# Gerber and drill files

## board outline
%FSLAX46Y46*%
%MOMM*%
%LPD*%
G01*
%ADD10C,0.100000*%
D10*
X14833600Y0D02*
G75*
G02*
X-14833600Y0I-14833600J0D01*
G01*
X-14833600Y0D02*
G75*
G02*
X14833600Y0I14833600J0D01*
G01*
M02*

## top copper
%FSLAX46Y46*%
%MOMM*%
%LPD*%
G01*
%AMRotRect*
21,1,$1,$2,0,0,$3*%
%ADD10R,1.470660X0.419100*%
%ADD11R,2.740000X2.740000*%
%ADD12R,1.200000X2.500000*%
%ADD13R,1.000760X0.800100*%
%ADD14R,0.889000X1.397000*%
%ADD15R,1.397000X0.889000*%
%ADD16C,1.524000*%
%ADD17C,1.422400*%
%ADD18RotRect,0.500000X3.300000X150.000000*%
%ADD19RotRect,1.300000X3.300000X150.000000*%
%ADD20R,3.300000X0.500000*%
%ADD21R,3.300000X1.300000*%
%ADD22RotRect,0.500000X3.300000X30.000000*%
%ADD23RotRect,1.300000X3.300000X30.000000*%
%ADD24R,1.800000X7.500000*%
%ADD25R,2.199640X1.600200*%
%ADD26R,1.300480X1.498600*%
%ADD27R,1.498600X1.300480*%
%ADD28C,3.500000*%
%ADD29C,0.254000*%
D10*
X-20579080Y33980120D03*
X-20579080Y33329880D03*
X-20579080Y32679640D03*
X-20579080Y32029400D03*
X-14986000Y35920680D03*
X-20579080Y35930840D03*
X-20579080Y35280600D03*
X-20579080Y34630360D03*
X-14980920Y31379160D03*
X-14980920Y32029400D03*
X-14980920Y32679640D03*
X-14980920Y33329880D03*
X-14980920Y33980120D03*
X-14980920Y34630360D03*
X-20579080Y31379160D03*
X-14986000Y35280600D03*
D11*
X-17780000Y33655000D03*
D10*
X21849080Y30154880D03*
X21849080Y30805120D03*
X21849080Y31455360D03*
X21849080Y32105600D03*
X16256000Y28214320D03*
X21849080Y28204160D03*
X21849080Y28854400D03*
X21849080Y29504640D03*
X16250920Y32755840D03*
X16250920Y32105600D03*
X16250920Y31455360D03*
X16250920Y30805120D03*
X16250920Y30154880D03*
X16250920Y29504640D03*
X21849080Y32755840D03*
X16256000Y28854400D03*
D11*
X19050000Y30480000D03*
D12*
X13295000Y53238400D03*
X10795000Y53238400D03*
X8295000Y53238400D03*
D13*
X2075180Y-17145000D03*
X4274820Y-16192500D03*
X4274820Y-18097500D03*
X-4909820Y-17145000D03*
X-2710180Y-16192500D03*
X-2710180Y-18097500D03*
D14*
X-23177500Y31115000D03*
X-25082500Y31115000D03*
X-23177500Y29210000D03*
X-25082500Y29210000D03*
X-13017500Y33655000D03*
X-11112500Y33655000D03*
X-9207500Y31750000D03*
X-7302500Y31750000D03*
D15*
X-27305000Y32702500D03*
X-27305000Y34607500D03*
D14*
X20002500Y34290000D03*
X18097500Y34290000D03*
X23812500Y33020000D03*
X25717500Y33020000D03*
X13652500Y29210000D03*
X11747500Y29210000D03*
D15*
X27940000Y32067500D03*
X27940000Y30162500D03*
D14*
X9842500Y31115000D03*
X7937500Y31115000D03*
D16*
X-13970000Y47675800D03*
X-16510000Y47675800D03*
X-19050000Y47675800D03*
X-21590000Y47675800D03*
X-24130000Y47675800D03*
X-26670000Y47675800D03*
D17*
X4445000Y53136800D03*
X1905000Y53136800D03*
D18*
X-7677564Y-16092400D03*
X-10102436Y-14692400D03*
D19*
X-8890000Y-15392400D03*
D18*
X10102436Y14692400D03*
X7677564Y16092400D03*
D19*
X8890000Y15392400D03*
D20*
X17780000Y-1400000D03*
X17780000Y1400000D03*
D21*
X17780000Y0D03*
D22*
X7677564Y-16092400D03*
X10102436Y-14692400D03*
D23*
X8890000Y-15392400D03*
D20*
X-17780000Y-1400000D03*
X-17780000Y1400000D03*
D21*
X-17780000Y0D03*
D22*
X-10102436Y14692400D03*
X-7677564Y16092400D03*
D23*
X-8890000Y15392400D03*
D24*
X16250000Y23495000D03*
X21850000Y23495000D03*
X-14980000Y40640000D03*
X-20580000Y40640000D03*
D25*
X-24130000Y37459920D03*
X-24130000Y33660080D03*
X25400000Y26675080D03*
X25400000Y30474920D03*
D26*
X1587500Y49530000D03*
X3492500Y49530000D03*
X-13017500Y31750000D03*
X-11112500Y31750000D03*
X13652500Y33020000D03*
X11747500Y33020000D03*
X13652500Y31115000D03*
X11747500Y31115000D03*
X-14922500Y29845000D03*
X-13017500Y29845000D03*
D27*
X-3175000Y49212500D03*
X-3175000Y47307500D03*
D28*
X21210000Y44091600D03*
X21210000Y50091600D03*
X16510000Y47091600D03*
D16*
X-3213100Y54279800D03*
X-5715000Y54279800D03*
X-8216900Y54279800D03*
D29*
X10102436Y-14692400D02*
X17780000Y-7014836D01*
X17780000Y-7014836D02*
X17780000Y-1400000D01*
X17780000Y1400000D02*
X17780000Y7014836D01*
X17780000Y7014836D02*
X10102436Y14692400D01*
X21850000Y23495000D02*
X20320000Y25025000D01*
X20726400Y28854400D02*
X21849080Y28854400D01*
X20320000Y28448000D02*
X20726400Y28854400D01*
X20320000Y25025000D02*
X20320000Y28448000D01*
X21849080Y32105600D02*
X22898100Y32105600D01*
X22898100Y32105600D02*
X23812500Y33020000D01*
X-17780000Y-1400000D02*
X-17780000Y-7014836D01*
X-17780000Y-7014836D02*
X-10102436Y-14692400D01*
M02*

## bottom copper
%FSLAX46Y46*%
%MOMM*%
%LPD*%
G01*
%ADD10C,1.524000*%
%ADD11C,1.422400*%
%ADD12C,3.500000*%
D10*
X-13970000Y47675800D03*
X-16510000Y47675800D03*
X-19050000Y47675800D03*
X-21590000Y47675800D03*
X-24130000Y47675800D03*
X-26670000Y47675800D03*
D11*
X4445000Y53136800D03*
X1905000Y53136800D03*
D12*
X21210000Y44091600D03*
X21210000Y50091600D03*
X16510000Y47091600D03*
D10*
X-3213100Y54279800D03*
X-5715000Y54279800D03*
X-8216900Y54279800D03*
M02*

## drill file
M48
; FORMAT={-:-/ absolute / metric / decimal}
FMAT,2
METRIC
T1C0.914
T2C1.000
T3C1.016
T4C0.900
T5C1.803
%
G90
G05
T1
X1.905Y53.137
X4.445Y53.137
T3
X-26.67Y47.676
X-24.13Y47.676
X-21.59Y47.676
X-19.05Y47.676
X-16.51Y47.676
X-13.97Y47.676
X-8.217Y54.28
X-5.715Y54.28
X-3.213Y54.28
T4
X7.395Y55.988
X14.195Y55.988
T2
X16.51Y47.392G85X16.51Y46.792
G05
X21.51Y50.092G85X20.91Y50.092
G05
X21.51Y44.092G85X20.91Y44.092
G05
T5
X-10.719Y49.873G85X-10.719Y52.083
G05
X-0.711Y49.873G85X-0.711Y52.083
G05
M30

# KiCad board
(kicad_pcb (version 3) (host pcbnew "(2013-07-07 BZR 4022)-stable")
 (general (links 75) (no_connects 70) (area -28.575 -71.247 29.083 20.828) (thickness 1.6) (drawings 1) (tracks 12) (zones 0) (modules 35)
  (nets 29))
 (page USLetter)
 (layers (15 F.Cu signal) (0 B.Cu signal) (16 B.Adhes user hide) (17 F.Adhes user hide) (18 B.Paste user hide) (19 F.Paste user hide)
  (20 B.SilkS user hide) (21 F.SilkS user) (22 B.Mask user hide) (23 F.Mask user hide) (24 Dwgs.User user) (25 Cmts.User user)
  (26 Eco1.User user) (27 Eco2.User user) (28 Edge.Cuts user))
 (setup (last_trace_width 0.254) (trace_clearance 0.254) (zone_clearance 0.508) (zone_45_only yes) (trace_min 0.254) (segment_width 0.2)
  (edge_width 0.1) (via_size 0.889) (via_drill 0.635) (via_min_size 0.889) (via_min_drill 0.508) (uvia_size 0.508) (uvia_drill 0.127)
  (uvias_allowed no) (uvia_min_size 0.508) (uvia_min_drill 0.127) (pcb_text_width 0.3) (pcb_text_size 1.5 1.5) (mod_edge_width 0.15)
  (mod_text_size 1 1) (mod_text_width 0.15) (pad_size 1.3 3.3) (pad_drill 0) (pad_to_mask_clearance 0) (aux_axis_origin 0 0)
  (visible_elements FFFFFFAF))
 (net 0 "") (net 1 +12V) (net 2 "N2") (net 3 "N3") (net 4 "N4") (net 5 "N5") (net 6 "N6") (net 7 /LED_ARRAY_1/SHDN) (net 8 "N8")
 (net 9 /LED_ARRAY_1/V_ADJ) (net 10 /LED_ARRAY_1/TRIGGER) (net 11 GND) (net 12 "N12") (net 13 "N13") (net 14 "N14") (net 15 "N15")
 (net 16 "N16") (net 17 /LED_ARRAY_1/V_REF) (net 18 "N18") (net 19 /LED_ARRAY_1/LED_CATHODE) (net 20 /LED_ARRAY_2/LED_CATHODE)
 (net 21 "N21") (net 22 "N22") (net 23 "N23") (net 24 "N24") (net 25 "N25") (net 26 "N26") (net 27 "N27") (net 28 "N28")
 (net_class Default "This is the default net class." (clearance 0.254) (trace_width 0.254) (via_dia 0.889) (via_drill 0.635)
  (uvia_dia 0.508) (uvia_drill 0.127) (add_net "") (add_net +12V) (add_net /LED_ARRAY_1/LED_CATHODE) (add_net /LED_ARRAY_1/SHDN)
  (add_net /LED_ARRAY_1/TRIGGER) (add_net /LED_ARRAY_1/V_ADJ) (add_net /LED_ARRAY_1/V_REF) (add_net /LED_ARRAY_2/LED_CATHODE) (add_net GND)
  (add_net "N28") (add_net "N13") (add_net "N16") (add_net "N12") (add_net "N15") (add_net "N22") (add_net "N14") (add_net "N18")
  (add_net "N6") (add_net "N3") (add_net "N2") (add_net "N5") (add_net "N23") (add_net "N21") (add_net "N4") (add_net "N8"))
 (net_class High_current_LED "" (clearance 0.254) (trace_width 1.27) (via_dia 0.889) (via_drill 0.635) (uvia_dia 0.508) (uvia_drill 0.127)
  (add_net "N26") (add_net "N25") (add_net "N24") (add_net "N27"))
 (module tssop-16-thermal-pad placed (layer F.Cu) (at -17.78 -33.655 270)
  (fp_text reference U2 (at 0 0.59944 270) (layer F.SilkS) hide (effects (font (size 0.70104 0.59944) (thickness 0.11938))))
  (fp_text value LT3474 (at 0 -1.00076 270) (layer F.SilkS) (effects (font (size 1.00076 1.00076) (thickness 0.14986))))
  (pad 4 smd rect (at -0.32512 2.79908 270) (size 0.4191 1.47066) (layers F.Cu F.Paste F.Mask) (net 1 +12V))
  (pad 5 smd rect (at 0.32512 2.79908 270) (size 0.4191 1.47066) (layers F.Cu F.Paste F.Mask) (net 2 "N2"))
  (pad 6 smd rect (at 0.97536 2.79908 270) (size 0.4191 1.47066) (layers F.Cu F.Paste F.Mask) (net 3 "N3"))
  (pad 7 smd rect (at 1.6256 2.79908 270) (size 0.4191 1.47066) (layers F.Cu F.Paste F.Mask) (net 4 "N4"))
  (pad 16 smd rect (at -2.26568 -2.794 270) (size 0.4191 1.47066) (layers F.Cu F.Paste F.Mask))
  (pad 1 smd rect (at -2.27584 2.79908 270) (size 0.4191 1.47066) (layers F.Cu F.Paste F.Mask))
  (pad 2 smd rect (at -1.6256 2.79908 270) (size 0.4191 1.47066) (layers F.Cu F.Paste F.Mask) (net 4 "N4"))
  (pad 3 smd rect (at -0.97536 2.79908 270) (size 0.4191 1.47066) (layers F.Cu F.Paste F.Mask) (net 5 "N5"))
  (pad 9 smd rect (at 2.27584 -2.79908 270) (size 0.4191 1.47066) (layers F.Cu F.Paste F.Mask) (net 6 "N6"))
  (pad 10 smd rect (at 1.6256 -2.79908 270) (size 0.4191 1.47066) (layers F.Cu F.Paste F.Mask) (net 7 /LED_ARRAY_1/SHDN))
  (pad 11 smd rect (at 0.97536 -2.79908 270) (size 0.4191 1.47066) (layers F.Cu F.Paste F.Mask))
  (pad 12 smd rect (at 0.32512 -2.79908 270) (size 0.4191 1.47066) (layers F.Cu F.Paste F.Mask) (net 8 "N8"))
  (pad 13 smd rect (at -0.32512 -2.79908 270) (size 0.4191 1.47066) (layers F.Cu F.Paste F.Mask) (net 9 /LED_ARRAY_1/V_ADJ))
  (pad 14 smd rect (at -0.97536 -2.79908 270) (size 0.4191 1.47066) (layers F.Cu F.Paste F.Mask) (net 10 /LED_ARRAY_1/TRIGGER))
  (pad 8 smd rect (at 2.27584 2.79908 270) (size 0.4191 1.47066) (layers F.Cu F.Paste F.Mask) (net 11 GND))
  (pad 15 smd rect (at -1.6256 -2.794 270) (size 0.4191 1.47066) (layers F.Cu F.Paste F.Mask) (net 11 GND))
  (pad 17 smd rect (at 0 0 270) (size 2.74 2.74) (layers F.Cu F.Paste F.Mask) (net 11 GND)))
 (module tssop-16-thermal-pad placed (layer F.Cu) (at 19.05 -30.48 90)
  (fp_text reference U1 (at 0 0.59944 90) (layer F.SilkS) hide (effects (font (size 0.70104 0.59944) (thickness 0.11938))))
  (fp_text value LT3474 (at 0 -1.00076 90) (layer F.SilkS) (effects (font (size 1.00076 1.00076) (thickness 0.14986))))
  (pad 4 smd rect (at -0.32512 2.79908 90) (size 0.4191 1.47066) (layers F.Cu F.Paste F.Mask) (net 1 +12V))
  (pad 5 smd rect (at 0.32512 2.79908 90) (size 0.4191 1.47066) (layers F.Cu F.Paste F.Mask) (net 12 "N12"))
  (pad 6 smd rect (at 0.97536 2.79908 90) (size 0.4191 1.47066) (layers F.Cu F.Paste F.Mask) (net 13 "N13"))
  (pad 7 smd rect (at 1.6256 2.79908 90) (size 0.4191 1.47066) (layers F.Cu F.Paste F.Mask) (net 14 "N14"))
  (pad 16 smd rect (at -2.26568 -2.794 90) (size 0.4191 1.47066) (layers F.Cu F.Paste F.Mask))
  (pad 1 smd rect (at -2.27584 2.79908 90) (size 0.4191 1.47066) (layers F.Cu F.Paste F.Mask))
  (pad 2 smd rect (at -1.6256 2.79908 90) (size 0.4191 1.47066) (layers F.Cu F.Paste F.Mask) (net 14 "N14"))
  (pad 3 smd rect (at -0.97536 2.79908 90) (size 0.4191 1.47066) (layers F.Cu F.Paste F.Mask) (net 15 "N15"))
  (pad 9 smd rect (at 2.27584 -2.79908 90) (size 0.4191 1.47066) (layers F.Cu F.Paste F.Mask) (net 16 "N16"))
  (pad 10 smd rect (at 1.6256 -2.79908 90) (size 0.4191 1.47066) (layers F.Cu F.Paste F.Mask) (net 7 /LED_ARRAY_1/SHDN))
  (pad 11 smd rect (at 0.97536 -2.79908 90) (size 0.4191 1.47066) (layers F.Cu F.Paste F.Mask) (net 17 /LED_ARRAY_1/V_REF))
  (pad 12 smd rect (at 0.32512 -2.79908 90) (size 0.4191 1.47066) (layers F.Cu F.Paste F.Mask) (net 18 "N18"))
  (pad 13 smd rect (at -0.32512 -2.79908 90) (size 0.4191 1.47066) (layers F.Cu F.Paste F.Mask) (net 9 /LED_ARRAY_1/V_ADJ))
  (pad 14 smd rect (at -0.97536 -2.79908 90) (size 0.4191 1.47066) (layers F.Cu F.Paste F.Mask) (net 10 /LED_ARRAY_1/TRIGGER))
  (pad 8 smd rect (at 2.27584 2.79908 90) (size 0.4191 1.47066) (layers F.Cu F.Paste F.Mask) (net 11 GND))
  (pad 15 smd rect (at -1.6256 -2.794 90) (size 0.4191 1.47066) (layers F.Cu F.Paste F.Mask) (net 11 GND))
  (pad 17 smd rect (at 0 0 90) (size 2.74 2.74) (layers F.Cu F.Paste F.Mask) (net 11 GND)))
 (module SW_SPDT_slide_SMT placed (layer F.Cu) (at 10.795 -53.2384 180)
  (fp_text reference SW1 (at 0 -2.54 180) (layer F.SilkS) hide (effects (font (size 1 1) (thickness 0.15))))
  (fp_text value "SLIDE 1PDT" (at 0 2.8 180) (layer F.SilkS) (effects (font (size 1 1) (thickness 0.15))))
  (pad 1 smd rect (at -2.5 0 180) (size 1.2 2.5) (layers F.Cu F.Paste F.Mask) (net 11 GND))
  (pad 2 smd rect (at 0 0 180) (size 1.2 2.5) (layers F.Cu F.Paste F.Mask) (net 7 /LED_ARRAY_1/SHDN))
  (pad 3 smd rect (at 2.5 0 180) (size 1.2 2.5) (layers F.Cu F.Paste F.Mask) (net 1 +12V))
  (pad "" np_thru_hole circle (at 3.4 2.75 180) (size 0.9 0.9) (drill 0.9) (layers *.Cu *.Mask F.SilkS))
  (pad "" np_thru_hole circle (at -3.4 2.75 180) (size 0.9 0.9) (drill 0.9) (layers *.Cu *.Mask F.SilkS)))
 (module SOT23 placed (layer F.Cu) (at 3.175 17.145 90)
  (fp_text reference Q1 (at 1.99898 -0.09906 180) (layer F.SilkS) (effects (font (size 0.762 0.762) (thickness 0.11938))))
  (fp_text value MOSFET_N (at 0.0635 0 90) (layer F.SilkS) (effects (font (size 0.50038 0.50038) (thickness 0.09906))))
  (pad 3 smd rect (at 0 -1.09982 90) (size 0.8001 1.00076) (layers F.Cu F.Paste F.Mask) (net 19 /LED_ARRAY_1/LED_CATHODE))
  (pad 2 smd rect (at 0.9525 1.09982 90) (size 0.8001 1.00076) (layers F.Cu F.Paste F.Mask) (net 11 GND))
  (pad 1 smd rect (at -0.9525 1.09982 90) (size 0.8001 1.00076) (layers F.Cu F.Paste F.Mask) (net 10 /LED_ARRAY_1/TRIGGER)))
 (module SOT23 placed (layer F.Cu) (at -3.81 17.145 90)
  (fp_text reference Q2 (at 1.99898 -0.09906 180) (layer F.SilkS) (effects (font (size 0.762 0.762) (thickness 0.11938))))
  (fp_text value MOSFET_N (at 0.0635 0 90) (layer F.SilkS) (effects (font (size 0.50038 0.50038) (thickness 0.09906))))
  (pad 3 smd rect (at 0 -1.09982 90) (size 0.8001 1.00076) (layers F.Cu F.Paste F.Mask) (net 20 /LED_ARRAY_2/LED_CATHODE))
  (pad 2 smd rect (at 0.9525 1.09982 90) (size 0.8001 1.00076) (layers F.Cu F.Paste F.Mask) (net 11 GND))
  (pad 1 smd rect (at -0.9525 1.09982 90) (size 0.8001 1.00076) (layers F.Cu F.Paste F.Mask) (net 10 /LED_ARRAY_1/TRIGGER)))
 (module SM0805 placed (layer F.Cu) (at -24.13 -31.115 180)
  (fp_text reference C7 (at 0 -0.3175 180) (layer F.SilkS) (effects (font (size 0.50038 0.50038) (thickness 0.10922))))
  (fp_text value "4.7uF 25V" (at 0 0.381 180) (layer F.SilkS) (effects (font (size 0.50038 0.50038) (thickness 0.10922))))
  (pad 1 smd rect (at -0.9525 0 180) (size 0.889 1.397) (layers F.Cu F.Paste F.Mask) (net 1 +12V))
  (pad 2 smd rect (at 0.9525 0 180) (size 0.889 1.397) (layers F.Cu F.Paste F.Mask) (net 11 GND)))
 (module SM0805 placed (layer F.Cu) (at -24.13 -29.21 180)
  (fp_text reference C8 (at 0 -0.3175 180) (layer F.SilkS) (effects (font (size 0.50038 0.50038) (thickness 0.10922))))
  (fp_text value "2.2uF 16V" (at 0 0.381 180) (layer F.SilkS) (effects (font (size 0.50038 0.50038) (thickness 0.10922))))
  (pad 1 smd rect (at -0.9525 0 180) (size 0.889 1.397) (layers F.Cu F.Paste F.Mask) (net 4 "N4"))
  (pad 2 smd rect (at 0.9525 0 180) (size 0.889 1.397) (layers F.Cu F.Paste F.Mask) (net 11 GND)))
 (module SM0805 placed (layer F.Cu) (at -12.065 -33.655)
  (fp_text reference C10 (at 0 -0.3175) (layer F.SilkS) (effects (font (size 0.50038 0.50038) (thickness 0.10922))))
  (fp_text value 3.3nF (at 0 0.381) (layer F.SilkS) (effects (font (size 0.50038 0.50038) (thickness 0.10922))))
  (pad 1 smd rect (at -0.9525 0) (size 0.889 1.397) (layers F.Cu F.Paste F.Mask) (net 8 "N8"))
  (pad 2 smd rect (at 0.9525 0) (size 0.889 1.397) (layers F.Cu F.Paste F.Mask) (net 11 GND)))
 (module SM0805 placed (layer F.Cu) (at -8.255 -31.75)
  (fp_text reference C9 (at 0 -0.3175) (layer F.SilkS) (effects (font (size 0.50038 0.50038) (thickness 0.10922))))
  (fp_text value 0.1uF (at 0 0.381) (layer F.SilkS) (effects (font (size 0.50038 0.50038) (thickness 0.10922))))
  (pad 1 smd rect (at -0.9525 0) (size 0.889 1.397) (layers F.Cu F.Paste F.Mask) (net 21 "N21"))
  (pad 2 smd rect (at 0.9525 0) (size 0.889 1.397) (layers F.Cu F.Paste F.Mask) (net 11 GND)))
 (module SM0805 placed (layer F.Cu) (at -27.305 -33.655 90)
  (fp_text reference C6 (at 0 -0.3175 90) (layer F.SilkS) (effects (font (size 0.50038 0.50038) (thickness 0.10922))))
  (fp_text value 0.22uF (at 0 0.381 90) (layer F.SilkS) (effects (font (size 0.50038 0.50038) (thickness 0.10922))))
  (pad 1 smd rect (at -0.9525 0 90) (size 0.889 1.397) (layers F.Cu F.Paste F.Mask) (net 3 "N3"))
  (pad 2 smd rect (at 0.9525 0 90) (size 0.889 1.397) (layers F.Cu F.Paste F.Mask) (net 2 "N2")))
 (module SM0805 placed (layer F.Cu) (at 19.05 -34.29 180)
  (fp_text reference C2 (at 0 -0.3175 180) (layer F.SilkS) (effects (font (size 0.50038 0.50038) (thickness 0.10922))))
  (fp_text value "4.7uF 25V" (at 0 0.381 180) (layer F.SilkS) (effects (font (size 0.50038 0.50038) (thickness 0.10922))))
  (pad 1 smd rect (at -0.9525 0 180) (size 0.889 1.397) (layers F.Cu F.Paste F.Mask) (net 1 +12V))
  (pad 2 smd rect (at 0.9525 0 180) (size 0.889 1.397) (layers F.Cu F.Paste F.Mask) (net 11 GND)))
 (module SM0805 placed (layer F.Cu) (at 24.765 -33.02)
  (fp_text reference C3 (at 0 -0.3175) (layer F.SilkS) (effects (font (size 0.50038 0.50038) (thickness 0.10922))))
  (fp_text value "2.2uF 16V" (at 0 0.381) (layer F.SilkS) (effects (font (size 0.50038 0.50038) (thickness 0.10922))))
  (pad 1 smd rect (at -0.9525 0) (size 0.889 1.397) (layers F.Cu F.Paste F.Mask) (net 14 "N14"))
  (pad 2 smd rect (at 0.9525 0) (size 0.889 1.397) (layers F.Cu F.Paste F.Mask) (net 11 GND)))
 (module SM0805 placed (layer F.Cu) (at 12.7 -29.21 180)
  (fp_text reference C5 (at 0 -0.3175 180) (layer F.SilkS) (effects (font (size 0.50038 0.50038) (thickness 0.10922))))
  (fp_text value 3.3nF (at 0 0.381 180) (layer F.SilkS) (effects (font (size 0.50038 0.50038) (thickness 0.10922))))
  (pad 1 smd rect (at -0.9525 0 180) (size 0.889 1.397) (layers F.Cu F.Paste F.Mask) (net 18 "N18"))
  (pad 2 smd rect (at 0.9525 0 180) (size 0.889 1.397) (layers F.Cu F.Paste F.Mask) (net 11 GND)))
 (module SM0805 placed (layer F.Cu) (at 27.94 -31.115 270)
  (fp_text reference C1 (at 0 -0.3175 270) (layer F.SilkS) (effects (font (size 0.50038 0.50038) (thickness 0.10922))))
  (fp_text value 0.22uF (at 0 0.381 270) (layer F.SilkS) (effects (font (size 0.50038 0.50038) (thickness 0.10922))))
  (pad 1 smd rect (at -0.9525 0 270) (size 0.889 1.397) (layers F.Cu F.Paste F.Mask) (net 13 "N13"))
  (pad 2 smd rect (at 0.9525 0 270) (size 0.889 1.397) (layers F.Cu F.Paste F.Mask) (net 12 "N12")))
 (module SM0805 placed (layer F.Cu) (at 8.89 -31.115 180)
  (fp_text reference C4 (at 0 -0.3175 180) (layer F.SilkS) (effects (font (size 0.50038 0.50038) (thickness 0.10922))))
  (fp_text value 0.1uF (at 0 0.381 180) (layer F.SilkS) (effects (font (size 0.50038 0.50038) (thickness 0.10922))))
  (pad 1 smd rect (at -0.9525 0 180) (size 0.889 1.397) (layers F.Cu F.Paste F.Mask) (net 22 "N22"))
  (pad 2 smd rect (at 0.9525 0 180) (size 0.889 1.397) (layers F.Cu F.Paste F.Mask) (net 11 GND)))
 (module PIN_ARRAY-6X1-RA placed (layer F.Cu) (at -20.32 -47.6758 180)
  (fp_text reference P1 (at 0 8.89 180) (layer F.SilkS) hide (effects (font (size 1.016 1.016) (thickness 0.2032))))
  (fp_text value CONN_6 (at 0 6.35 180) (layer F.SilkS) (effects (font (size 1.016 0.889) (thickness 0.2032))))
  (pad 1 thru_hole circle (at -6.35 0 180) (size 1.524 1.524) (drill 1.016) (layers *.Cu *.Mask F.SilkS) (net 11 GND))
  (pad 2 thru_hole circle (at -3.81 0 180) (size 1.524 1.524) (drill 1.016) (layers *.Cu *.Mask F.SilkS) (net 9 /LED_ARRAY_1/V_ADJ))
  (pad 3 thru_hole circle (at -1.27 0 180) (size 1.524 1.524) (drill 1.016) (layers *.Cu *.Mask F.SilkS) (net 17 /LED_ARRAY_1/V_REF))
  (pad 4 thru_hole circle (at 1.27 0 180) (size 1.524 1.524) (drill 1.016) (layers *.Cu *.Mask F.SilkS) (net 10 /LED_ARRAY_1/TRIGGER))
  (pad 5 thru_hole circle (at 3.81 0 180) (size 1.524 1.524) (drill 1.016) (layers *.Cu *.Mask F.SilkS))
  (pad 6 thru_hole circle (at 6.35 0 180) (size 1.524 1.524) (drill 1.016) (layers *.Cu *.Mask F.SilkS) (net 1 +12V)))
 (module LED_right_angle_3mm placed (layer F.Cu) (at 4.445 -53.1368 180)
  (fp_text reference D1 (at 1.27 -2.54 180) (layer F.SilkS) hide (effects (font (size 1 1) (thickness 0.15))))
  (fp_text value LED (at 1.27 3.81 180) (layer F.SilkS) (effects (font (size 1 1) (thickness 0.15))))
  (pad 1 thru_hole circle (at 0 0 180) (size 1.4224 1.4224) (drill 0.9144) (layers *.Cu *.Mask F.SilkS) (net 7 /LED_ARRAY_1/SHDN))
  (pad 2 thru_hole circle (at 2.54 0 180) (size 1.4224 1.4224) (drill 0.9144) (layers *.Cu *.Mask F.SilkS) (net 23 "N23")))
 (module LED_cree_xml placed (layer F.Cu) (at -8.89 15.3924 150)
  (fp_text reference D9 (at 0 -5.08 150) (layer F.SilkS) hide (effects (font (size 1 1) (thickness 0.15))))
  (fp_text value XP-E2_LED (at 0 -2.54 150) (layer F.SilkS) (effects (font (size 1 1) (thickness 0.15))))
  (pad 2 smd rect (at -1.4 0 150) (size 0.5 3.3) (layers F.Cu F.Paste F.Mask) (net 20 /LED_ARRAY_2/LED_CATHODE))
  (pad 1 smd rect (at 1.4 0 150) (size 0.5 3.3) (layers F.Cu F.Paste F.Mask) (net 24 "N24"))
  (pad 3 smd rect (at 0 0 150) (size 1.3 3.3) (layers F.Cu F.Paste F.Mask)))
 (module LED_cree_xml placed (layer F.Cu) (at 8.89 -15.3924 150)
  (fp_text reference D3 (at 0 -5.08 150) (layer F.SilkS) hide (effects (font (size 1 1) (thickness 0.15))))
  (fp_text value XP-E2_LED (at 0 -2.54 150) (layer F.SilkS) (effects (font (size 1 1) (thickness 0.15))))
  (pad 2 smd rect (at -1.4 0 150) (size 0.5 3.3) (layers F.Cu F.Paste F.Mask) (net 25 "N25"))
  (pad 1 smd rect (at 1.4 0 150) (size 0.5 3.3) (layers F.Cu F.Paste F.Mask) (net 15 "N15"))
  (pad 3 smd rect (at 0 0 150) (size 1.3 3.3) (layers F.Cu F.Paste F.Mask)))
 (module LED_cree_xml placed (layer F.Cu) (at 17.78 0 90)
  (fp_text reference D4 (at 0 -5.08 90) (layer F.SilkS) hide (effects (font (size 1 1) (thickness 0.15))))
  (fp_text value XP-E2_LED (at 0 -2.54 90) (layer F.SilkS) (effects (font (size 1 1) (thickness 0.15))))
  (pad 2 smd rect (at -1.4 0 90) (size 0.5 3.3) (layers F.Cu F.Paste F.Mask) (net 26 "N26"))
  (pad 1 smd rect (at 1.4 0 90) (size 0.5 3.3) (layers F.Cu F.Paste F.Mask) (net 25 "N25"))
  (pad 3 smd rect (at 0 0 90) (size 1.3 3.3) (layers F.Cu F.Paste F.Mask)))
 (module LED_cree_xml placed (layer F.Cu) (at 8.89 15.3924 30)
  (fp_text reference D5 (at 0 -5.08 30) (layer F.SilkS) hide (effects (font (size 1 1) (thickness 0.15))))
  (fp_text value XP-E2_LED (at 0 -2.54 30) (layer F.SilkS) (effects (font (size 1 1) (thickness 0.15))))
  (pad 2 smd rect (at -1.4 0 30) (size 0.5 3.3) (layers F.Cu F.Paste F.Mask) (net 19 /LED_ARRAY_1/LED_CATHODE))
  (pad 1 smd rect (at 1.4 0 30) (size 0.5 3.3) (layers F.Cu F.Paste F.Mask) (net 26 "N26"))
  (pad 3 smd rect (at 0 0 30) (size 1.3 3.3) (layers F.Cu F.Paste F.Mask)))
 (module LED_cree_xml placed (layer F.Cu) (at -17.78 0 90)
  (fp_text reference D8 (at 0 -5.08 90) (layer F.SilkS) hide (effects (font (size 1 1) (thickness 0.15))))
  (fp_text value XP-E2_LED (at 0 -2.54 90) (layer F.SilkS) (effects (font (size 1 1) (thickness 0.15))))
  (pad 2 smd rect (at -1.4 0 90) (size 0.5 3.3) (layers F.Cu F.Paste F.Mask) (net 24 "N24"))
  (pad 1 smd rect (at 1.4 0 90) (size 0.5 3.3) (layers F.Cu F.Paste F.Mask) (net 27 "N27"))
  (pad 3 smd rect (at 0 0 90) (size 1.3 3.3) (layers F.Cu F.Paste F.Mask)))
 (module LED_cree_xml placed (layer F.Cu) (at -8.89 -15.3924 30)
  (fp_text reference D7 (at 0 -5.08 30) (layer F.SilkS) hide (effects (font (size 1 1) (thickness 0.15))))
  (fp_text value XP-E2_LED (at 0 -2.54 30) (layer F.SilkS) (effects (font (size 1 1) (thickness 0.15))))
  (pad 2 smd rect (at -1.4 0 30) (size 0.5 3.3) (layers F.Cu F.Paste F.Mask) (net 27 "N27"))
  (pad 1 smd rect (at 1.4 0 30) (size 0.5 3.3) (layers F.Cu F.Paste F.Mask) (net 5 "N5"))
  (pad 3 smd rect (at 0 0 30) (size 1.3 3.3) (layers F.Cu F.Paste F.Mask)))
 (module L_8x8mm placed (layer F.Cu) (at 19.05 -23.495)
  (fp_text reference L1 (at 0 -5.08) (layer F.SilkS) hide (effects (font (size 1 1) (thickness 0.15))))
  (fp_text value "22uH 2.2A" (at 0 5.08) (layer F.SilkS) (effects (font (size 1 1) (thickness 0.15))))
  (pad 1 smd rect (at -2.8 0) (size 1.8 7.5) (layers F.Cu F.Paste F.Mask) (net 12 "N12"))
  (pad 2 smd rect (at 2.8 0) (size 1.8 7.5) (layers F.Cu F.Paste F.Mask) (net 14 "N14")))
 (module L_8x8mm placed (layer F.Cu) (at -17.78 -40.64 180)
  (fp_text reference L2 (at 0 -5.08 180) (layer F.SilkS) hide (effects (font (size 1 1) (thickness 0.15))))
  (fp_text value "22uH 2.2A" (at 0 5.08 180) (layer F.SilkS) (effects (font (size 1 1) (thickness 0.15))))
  (pad 1 smd rect (at -2.8 0 180) (size 1.8 7.5) (layers F.Cu F.Paste F.Mask) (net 2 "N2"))
  (pad 2 smd rect (at 2.8 0 180) (size 1.8 7.5) (layers F.Cu F.Paste F.Mask) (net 4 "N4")))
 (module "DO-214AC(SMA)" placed (layer F.Cu) (at -24.13 -35.56 270)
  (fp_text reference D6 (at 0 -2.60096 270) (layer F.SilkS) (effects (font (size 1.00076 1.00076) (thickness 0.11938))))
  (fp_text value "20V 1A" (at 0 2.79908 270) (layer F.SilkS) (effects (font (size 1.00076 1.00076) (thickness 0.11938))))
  (pad 1 smd rect (at -1.89992 0 270) (size 1.6002 2.19964) (layers F.Cu F.Paste F.Mask) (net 11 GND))
  (pad 2 smd rect (at 1.89992 0 270) (size 1.6002 2.19964) (layers F.Cu F.Paste F.Mask) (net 2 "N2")))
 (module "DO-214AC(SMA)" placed (layer F.Cu) (at 25.4 -28.575 90)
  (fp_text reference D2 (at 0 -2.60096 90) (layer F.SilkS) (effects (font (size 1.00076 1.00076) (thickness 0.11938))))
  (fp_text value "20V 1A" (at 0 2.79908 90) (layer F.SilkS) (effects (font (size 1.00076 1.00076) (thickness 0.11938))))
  (pad 1 smd rect (at -1.89992 0 90) (size 1.6002 2.19964) (layers F.Cu F.Paste F.Mask) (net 11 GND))
  (pad 2 smd rect (at 1.89992 0 90) (size 1.6002 2.19964) (layers F.Cu F.Paste F.Mask) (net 12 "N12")))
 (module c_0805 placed (layer F.Cu) (at 2.54 -49.53 180)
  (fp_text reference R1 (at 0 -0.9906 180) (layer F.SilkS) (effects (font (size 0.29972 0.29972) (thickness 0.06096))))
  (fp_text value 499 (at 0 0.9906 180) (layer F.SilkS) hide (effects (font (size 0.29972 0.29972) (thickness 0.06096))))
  (pad 1 smd rect (at 0.9525 0 180) (size 1.30048 1.4986) (layers F.Cu F.Paste F.Mask) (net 23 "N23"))
  (pad 2 smd rect (at -0.9525 0 180) (size 1.30048 1.4986) (layers F.Cu F.Paste F.Mask) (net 11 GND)))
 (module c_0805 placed (layer F.Cu) (at -12.065 -31.75 180)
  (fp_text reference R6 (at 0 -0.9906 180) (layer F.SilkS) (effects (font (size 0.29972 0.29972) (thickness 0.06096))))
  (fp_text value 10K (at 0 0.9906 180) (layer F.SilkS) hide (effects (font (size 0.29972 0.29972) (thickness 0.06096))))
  (pad 1 smd rect (at 0.9525 0 180) (size 1.30048 1.4986) (layers F.Cu F.Paste F.Mask) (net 8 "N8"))
  (pad 2 smd rect (at -0.9525 0 180) (size 1.30048 1.4986) (layers F.Cu F.Paste F.Mask) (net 21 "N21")))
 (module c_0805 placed (layer F.Cu) (at 12.7 -33.02)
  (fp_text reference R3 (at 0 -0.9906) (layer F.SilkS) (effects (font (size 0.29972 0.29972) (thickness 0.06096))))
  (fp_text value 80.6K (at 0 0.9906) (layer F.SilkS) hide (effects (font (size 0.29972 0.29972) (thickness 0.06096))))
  (pad 1 smd rect (at 0.9525 0) (size 1.30048 1.4986) (layers F.Cu F.Paste F.Mask) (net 16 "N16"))
  (pad 2 smd rect (at -0.9525 0) (size 1.30048 1.4986) (layers F.Cu F.Paste F.Mask) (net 11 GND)))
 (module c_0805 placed (layer F.Cu) (at 12.7 -31.115)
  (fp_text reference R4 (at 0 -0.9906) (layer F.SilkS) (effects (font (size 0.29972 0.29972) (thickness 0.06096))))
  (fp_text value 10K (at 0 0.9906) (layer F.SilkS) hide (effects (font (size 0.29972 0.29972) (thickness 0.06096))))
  (pad 1 smd rect (at 0.9525 0) (size 1.30048 1.4986) (layers F.Cu F.Paste F.Mask) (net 18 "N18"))
  (pad 2 smd rect (at -0.9525 0) (size 1.30048 1.4986) (layers F.Cu F.Paste F.Mask) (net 22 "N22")))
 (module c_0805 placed (layer F.Cu) (at -13.97 -29.845 180)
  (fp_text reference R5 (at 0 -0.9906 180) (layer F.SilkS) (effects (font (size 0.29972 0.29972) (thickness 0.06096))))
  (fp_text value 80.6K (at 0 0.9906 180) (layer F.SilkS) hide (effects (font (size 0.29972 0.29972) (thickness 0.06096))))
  (pad 1 smd rect (at 0.9525 0 180) (size 1.30048 1.4986) (layers F.Cu F.Paste F.Mask) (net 6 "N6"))
  (pad 2 smd rect (at -0.9525 0 180) (size 1.30048 1.4986) (layers F.Cu F.Paste F.Mask) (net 11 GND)))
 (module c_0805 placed (layer F.Cu) (at -3.175 -48.26 90)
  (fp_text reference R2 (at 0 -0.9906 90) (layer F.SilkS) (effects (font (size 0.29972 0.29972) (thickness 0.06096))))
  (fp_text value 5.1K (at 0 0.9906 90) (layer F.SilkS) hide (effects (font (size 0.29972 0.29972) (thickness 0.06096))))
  (pad 1 smd rect (at 0.9525 0 90) (size 1.30048 1.4986) (layers F.Cu F.Paste F.Mask) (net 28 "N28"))
  (pad 2 smd rect (at -0.9525 0 90) (size 1.30048 1.4986) (layers F.Cu F.Paste F.Mask) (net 11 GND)))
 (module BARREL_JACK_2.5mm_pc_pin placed (layer F.Cu) (at 16.51 -47.0916)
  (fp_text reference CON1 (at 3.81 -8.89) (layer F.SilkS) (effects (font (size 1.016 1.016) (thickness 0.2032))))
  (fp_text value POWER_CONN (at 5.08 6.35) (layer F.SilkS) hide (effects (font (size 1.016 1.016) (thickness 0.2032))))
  (pad 1 thru_hole circle (at 4.7 3 270) (size 3.5 3.5) (drill oval 1 1.6) (layers *.Cu *.Mask F.SilkS) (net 1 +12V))
  (pad 2 thru_hole circle (at 4.7 -3 270) (size 3.5 3.5) (drill oval 1 1.6) (layers *.Cu *.Mask F.SilkS) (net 11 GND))
  (pad 3 thru_hole circle (at 0 0) (size 3.5 3.5) (drill oval 1 1.6) (layers *.Cu *.Mask F.SilkS) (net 11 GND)))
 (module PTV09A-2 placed (layer F.Cu) (at -5.715 -54.2798 180)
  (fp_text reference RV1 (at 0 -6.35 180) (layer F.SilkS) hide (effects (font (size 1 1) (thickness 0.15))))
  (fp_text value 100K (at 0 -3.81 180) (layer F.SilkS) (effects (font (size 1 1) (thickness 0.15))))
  (pad 1 thru_hole circle (at -2.5019 0 180) (size 1.524 1.524) (drill 1.016) (layers *.Cu *.Mask F.SilkS) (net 28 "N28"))
  (pad 2 thru_hole circle (at 0 0 180) (size 1.524 1.524) (drill 1.016) (layers *.Cu *.Mask F.SilkS) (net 9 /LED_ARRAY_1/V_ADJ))
  (pad 3 thru_hole circle (at 2.5019 0 180) (size 1.524 1.524) (drill 1.016) (layers *.Cu *.Mask F.SilkS) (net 17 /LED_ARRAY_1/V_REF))
  (pad "" np_thru_hole oval (at -5.0038 -3.302 180) (size 1.8034 4.0132) (drill oval 1.8034 4.0132) (layers *.Cu *.Mask F.SilkS))
  (pad "" np_thru_hole oval (at 5.0038 -3.302 180) (size 1.8034 4.0132) (drill oval 1.8034 4.0132) (layers *.Cu *.Mask F.SilkS)))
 (gr_circle (center 0 0) (end 0 14.8336) (layer Edge.Cuts) (width 0.1))
 (segment (start 10.102436 14.6924) (end 17.78 7.014836) (width 0.254) (layer F.Cu) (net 26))
 (segment (start 17.78 7.014836) (end 17.78 1.4) (width 0.254) (layer F.Cu) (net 26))
 (segment (start 17.78 -1.4) (end 17.78 -7.014836) (width 0.254) (layer F.Cu) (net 25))
 (segment (start 17.78 -7.014836) (end 10.102436 -14.6924) (width 0.254) (layer F.Cu) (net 25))
 (segment (start 21.85 -23.495) (end 20.32 -25.025) (width 0.254) (layer F.Cu) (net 14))
 (segment (start 20.7264 -28.8544) (end 21.84908 -28.8544) (width 0.254) (layer F.Cu) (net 14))
 (segment (start 20.32 -28.448) (end 20.7264 -28.8544) (width 0.254) (layer F.Cu) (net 14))
 (segment (start 20.32 -25.025) (end 20.32 -28.448) (width 0.254) (layer F.Cu) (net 14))
 (segment (start 21.84908 -32.1056) (end 22.8981 -32.1056) (width 0.254) (layer F.Cu) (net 14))
 (segment (start 22.8981 -32.1056) (end 23.8125 -33.02) (width 0.254) (layer F.Cu) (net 14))
 (segment (start -17.78 1.4) (end -17.78 7.014836) (width 0.254) (layer F.Cu) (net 24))
 (segment (start -17.78 7.014836) (end -10.102436 14.6924) (width 0.254) (layer F.Cu) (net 24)))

